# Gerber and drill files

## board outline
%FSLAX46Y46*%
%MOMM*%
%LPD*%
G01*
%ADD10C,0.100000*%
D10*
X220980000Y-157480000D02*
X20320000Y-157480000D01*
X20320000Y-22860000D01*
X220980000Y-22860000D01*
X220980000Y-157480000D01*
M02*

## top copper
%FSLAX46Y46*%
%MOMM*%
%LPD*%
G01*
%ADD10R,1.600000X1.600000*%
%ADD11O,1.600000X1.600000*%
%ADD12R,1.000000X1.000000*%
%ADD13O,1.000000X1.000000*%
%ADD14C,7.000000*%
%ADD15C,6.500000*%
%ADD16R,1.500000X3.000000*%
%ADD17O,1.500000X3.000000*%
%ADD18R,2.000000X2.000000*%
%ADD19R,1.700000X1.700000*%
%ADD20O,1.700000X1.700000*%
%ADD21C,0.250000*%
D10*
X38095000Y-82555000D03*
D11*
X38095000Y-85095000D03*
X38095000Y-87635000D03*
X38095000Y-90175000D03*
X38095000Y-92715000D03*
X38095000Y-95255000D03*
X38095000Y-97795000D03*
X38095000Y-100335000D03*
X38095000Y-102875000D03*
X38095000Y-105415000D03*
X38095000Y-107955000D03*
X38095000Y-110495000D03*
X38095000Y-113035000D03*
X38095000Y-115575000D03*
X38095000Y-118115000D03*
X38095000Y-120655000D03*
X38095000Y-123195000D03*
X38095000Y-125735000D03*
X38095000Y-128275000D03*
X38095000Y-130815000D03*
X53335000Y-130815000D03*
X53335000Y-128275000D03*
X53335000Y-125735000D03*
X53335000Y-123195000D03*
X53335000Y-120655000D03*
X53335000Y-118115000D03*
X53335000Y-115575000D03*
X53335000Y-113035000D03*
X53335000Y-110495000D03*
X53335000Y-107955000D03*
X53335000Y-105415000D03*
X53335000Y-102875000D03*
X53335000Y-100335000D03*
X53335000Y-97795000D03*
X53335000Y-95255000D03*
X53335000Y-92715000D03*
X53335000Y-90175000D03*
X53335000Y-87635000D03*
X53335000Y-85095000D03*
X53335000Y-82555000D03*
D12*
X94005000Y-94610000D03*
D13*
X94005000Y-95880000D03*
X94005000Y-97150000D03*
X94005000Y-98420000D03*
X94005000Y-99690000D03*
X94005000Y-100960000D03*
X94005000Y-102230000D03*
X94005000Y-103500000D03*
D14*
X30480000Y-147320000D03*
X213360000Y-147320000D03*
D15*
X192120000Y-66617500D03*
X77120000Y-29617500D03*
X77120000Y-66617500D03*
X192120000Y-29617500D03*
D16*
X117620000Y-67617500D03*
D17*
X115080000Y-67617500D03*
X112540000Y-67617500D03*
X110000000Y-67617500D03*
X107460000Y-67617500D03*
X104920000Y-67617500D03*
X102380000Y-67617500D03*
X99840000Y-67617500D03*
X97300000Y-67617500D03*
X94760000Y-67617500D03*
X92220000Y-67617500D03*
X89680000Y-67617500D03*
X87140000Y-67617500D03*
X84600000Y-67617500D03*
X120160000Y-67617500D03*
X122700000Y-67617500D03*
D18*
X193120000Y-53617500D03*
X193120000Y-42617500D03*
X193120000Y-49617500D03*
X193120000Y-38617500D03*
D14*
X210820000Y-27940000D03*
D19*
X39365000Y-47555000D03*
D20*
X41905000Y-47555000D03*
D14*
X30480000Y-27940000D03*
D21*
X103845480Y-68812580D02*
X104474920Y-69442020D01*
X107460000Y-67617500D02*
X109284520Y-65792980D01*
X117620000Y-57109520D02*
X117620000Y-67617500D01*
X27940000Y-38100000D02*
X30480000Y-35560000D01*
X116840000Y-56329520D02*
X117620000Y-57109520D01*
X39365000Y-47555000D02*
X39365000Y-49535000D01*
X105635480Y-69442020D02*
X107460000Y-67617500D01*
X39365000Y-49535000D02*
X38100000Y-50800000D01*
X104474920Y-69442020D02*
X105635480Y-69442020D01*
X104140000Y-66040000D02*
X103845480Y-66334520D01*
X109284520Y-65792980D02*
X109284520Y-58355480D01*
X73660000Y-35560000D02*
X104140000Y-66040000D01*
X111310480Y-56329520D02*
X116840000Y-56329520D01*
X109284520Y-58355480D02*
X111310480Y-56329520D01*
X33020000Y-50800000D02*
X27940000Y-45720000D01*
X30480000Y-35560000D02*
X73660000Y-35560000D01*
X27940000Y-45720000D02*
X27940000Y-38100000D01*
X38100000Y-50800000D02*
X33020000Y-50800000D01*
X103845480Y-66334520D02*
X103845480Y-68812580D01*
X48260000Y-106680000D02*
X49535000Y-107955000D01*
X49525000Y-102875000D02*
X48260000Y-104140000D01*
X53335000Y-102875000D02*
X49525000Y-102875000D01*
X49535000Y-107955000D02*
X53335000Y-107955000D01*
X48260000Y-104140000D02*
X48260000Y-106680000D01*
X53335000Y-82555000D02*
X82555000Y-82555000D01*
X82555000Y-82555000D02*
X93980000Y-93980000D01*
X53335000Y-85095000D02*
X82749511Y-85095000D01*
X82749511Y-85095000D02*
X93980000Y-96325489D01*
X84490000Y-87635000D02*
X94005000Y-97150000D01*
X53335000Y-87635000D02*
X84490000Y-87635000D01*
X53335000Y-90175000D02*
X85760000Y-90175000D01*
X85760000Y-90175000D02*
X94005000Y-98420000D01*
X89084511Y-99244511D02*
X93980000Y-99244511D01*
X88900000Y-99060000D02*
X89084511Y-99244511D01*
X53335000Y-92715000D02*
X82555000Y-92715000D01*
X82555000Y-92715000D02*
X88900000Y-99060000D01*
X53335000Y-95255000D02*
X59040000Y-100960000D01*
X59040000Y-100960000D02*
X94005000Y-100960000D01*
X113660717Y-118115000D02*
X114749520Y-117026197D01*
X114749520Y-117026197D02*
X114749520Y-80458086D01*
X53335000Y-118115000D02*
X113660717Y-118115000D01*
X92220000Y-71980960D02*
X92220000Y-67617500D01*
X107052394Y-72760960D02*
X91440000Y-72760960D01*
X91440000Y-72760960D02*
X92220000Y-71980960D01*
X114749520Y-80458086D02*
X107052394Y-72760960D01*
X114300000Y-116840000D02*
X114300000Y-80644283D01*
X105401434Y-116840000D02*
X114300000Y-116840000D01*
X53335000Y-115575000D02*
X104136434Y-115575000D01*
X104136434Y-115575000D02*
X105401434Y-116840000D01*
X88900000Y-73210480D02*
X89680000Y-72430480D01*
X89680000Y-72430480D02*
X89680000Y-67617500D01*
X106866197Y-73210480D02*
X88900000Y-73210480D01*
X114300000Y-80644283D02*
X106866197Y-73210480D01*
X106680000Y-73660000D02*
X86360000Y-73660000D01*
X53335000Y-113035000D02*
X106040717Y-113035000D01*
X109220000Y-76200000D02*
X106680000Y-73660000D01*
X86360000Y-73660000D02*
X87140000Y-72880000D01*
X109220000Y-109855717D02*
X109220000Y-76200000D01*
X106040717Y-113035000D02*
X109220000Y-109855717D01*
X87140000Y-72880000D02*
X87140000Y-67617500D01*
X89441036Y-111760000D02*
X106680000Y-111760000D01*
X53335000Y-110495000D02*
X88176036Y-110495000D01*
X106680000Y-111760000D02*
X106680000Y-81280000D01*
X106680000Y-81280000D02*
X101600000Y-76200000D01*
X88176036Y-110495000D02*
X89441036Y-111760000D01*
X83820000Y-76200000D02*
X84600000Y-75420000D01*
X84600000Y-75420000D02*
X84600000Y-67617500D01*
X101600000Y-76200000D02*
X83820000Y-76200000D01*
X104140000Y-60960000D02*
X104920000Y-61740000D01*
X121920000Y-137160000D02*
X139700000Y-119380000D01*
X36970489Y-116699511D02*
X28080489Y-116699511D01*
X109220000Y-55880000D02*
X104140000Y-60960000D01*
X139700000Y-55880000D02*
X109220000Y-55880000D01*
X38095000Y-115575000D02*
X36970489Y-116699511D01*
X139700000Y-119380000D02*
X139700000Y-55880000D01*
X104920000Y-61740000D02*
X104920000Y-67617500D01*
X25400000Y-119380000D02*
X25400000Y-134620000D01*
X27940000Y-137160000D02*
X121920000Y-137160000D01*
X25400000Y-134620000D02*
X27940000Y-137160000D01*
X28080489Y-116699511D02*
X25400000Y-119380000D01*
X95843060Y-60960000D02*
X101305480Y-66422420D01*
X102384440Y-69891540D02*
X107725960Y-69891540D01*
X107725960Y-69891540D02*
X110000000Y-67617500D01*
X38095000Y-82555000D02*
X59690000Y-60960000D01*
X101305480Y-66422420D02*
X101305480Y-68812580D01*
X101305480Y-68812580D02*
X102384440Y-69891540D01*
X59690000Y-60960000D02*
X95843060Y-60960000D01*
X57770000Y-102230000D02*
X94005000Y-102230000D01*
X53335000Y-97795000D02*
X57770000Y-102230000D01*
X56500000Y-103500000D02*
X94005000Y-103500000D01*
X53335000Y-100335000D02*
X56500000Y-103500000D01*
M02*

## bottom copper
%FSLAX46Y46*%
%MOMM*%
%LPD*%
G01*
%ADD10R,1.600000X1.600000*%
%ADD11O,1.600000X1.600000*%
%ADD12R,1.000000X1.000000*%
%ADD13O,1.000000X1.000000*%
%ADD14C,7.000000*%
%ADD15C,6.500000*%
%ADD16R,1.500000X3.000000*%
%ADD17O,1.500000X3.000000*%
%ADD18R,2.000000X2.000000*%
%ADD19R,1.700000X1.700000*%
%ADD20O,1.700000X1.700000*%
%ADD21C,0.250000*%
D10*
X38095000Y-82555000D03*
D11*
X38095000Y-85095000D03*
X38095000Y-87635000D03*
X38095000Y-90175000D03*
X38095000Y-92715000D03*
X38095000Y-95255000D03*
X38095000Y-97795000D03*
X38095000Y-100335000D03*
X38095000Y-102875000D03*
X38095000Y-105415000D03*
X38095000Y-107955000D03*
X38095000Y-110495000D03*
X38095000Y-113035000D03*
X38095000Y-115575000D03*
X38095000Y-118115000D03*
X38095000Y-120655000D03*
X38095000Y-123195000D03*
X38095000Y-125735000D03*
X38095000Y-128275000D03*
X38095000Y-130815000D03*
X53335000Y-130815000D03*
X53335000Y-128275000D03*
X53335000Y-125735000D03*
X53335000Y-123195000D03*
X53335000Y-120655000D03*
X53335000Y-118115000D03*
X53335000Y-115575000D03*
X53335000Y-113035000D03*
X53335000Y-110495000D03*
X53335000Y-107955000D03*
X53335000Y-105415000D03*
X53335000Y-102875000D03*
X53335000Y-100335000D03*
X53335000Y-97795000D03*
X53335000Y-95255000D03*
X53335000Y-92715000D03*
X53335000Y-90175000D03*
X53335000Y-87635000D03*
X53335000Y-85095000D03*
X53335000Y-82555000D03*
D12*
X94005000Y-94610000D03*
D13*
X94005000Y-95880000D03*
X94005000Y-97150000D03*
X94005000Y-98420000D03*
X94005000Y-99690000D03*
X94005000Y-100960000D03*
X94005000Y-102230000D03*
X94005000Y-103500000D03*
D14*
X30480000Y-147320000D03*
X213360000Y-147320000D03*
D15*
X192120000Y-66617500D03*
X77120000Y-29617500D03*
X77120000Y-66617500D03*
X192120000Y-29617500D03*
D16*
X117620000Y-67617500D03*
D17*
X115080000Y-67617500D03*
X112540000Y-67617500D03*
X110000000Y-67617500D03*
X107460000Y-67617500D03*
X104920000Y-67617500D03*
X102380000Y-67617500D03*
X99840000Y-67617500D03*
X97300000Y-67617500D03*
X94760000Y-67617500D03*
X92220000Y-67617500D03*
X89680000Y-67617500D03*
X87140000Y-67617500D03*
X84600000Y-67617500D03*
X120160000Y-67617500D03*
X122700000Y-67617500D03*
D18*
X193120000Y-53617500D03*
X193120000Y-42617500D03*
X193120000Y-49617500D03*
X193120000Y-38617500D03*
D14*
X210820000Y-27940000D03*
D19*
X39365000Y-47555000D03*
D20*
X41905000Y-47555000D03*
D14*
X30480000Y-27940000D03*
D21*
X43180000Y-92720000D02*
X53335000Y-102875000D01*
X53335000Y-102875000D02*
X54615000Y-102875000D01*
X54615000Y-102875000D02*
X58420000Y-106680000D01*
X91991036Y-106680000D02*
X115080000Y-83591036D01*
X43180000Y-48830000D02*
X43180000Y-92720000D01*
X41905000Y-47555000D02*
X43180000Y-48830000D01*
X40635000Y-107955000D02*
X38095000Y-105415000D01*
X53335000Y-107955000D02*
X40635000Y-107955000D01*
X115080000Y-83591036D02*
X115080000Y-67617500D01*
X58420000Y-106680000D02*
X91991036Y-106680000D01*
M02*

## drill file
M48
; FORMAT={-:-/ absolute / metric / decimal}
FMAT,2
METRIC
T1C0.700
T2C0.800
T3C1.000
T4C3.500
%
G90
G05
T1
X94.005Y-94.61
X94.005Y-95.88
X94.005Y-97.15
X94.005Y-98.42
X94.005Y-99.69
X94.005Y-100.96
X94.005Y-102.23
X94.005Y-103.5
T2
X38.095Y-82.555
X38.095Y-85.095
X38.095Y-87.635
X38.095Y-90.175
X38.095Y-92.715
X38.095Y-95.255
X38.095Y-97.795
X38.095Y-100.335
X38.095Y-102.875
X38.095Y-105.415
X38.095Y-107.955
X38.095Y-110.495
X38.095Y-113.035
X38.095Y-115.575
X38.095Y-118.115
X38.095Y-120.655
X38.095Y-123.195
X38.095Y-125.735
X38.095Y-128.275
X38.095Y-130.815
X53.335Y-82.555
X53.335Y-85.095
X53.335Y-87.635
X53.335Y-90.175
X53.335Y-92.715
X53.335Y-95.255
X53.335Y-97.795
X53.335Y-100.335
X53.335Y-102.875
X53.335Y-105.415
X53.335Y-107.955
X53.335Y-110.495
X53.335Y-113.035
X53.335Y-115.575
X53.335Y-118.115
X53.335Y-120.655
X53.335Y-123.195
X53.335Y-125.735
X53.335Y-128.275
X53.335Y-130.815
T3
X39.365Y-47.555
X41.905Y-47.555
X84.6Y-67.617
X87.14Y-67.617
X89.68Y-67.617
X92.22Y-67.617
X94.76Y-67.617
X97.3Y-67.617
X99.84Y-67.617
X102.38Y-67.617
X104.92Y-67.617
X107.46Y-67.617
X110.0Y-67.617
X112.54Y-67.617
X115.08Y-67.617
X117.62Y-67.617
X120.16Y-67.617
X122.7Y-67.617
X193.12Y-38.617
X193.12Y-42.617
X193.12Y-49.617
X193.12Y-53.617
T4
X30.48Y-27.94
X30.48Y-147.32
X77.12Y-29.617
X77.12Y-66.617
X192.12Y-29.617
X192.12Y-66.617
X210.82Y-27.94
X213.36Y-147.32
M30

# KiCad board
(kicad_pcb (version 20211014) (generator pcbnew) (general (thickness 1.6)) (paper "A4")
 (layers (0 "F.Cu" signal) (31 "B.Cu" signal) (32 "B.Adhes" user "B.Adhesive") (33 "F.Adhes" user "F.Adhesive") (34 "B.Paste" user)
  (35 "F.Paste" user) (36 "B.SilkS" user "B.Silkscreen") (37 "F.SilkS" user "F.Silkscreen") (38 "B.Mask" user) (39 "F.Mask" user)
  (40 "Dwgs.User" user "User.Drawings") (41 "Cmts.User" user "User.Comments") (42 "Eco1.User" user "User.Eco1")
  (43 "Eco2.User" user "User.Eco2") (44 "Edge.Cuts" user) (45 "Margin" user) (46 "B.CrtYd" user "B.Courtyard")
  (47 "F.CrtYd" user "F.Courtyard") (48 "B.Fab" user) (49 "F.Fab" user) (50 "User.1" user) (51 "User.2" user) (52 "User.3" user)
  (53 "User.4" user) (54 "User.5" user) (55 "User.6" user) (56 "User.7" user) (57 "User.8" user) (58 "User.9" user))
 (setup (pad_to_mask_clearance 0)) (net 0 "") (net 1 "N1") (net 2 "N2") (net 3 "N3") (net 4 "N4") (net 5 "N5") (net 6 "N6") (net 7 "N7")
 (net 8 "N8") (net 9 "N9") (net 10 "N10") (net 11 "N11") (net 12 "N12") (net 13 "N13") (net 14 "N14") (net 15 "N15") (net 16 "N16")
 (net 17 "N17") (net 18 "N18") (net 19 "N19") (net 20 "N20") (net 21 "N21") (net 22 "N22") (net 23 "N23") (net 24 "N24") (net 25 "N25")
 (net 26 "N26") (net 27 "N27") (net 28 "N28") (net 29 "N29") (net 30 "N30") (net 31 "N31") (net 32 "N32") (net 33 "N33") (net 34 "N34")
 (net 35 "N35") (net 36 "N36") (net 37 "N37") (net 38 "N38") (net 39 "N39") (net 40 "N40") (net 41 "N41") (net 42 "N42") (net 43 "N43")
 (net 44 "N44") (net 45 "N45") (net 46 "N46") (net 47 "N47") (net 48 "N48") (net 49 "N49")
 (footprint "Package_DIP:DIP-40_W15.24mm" (layer "F.Cu") (at 38.095 82.555)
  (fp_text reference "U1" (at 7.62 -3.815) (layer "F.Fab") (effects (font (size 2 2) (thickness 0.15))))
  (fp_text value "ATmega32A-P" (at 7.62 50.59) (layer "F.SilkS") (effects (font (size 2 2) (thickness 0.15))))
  (pad "1" thru_hole rect (at 0 0) (size 1.6 1.6) (drill 0.8) (layers *.Cu *.Mask) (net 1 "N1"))
  (pad "2" thru_hole oval (at 0 2.54) (size 1.6 1.6) (drill 0.8) (layers *.Cu *.Mask) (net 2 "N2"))
  (pad "3" thru_hole oval (at 0 5.08) (size 1.6 1.6) (drill 0.8) (layers *.Cu *.Mask) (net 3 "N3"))
  (pad "4" thru_hole oval (at 0 7.62) (size 1.6 1.6) (drill 0.8) (layers *.Cu *.Mask) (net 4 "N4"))
  (pad "5" thru_hole oval (at 0 10.16) (size 1.6 1.6) (drill 0.8) (layers *.Cu *.Mask) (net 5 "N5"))
  (pad "6" thru_hole oval (at 0 12.7) (size 1.6 1.6) (drill 0.8) (layers *.Cu *.Mask) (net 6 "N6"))
  (pad "7" thru_hole oval (at 0 15.24) (size 1.6 1.6) (drill 0.8) (layers *.Cu *.Mask) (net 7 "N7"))
  (pad "8" thru_hole oval (at 0 17.78) (size 1.6 1.6) (drill 0.8) (layers *.Cu *.Mask) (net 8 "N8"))
  (pad "9" thru_hole oval (at 0 20.32) (size 1.6 1.6) (drill 0.8) (layers *.Cu *.Mask) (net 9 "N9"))
  (pad "10" thru_hole oval (at 0 22.86) (size 1.6 1.6) (drill 0.8) (layers *.Cu *.Mask) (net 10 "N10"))
  (pad "11" thru_hole oval (at 0 25.4) (size 1.6 1.6) (drill 0.8) (layers *.Cu *.Mask) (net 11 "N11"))
  (pad "12" thru_hole oval (at 0 27.94) (size 1.6 1.6) (drill 0.8) (layers *.Cu *.Mask) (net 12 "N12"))
  (pad "13" thru_hole oval (at 0 30.48) (size 1.6 1.6) (drill 0.8) (layers *.Cu *.Mask) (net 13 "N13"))
  (pad "14" thru_hole oval (at 0 33.02) (size 1.6 1.6) (drill 0.8) (layers *.Cu *.Mask) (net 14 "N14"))
  (pad "15" thru_hole oval (at 0 35.56) (size 1.6 1.6) (drill 0.8) (layers *.Cu *.Mask) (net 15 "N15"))
  (pad "16" thru_hole oval (at 0 38.1) (size 1.6 1.6) (drill 0.8) (layers *.Cu *.Mask) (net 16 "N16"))
  (pad "17" thru_hole oval (at 0 40.64) (size 1.6 1.6) (drill 0.8) (layers *.Cu *.Mask) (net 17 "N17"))
  (pad "18" thru_hole oval (at 0 43.18) (size 1.6 1.6) (drill 0.8) (layers *.Cu *.Mask) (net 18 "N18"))
  (pad "19" thru_hole oval (at 0 45.72) (size 1.6 1.6) (drill 0.8) (layers *.Cu *.Mask) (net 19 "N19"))
  (pad "20" thru_hole oval (at 0 48.26) (size 1.6 1.6) (drill 0.8) (layers *.Cu *.Mask) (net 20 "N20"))
  (pad "21" thru_hole oval (at 15.24 48.26) (size 1.6 1.6) (drill 0.8) (layers *.Cu *.Mask) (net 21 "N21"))
  (pad "22" thru_hole oval (at 15.24 45.72) (size 1.6 1.6) (drill 0.8) (layers *.Cu *.Mask) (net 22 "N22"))
  (pad "23" thru_hole oval (at 15.24 43.18) (size 1.6 1.6) (drill 0.8) (layers *.Cu *.Mask) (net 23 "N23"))
  (pad "24" thru_hole oval (at 15.24 40.64) (size 1.6 1.6) (drill 0.8) (layers *.Cu *.Mask) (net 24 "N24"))
  (pad "25" thru_hole oval (at 15.24 38.1) (size 1.6 1.6) (drill 0.8) (layers *.Cu *.Mask) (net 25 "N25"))
  (pad "26" thru_hole oval (at 15.24 35.56) (size 1.6 1.6) (drill 0.8) (layers *.Cu *.Mask) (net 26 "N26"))
  (pad "27" thru_hole oval (at 15.24 33.02) (size 1.6 1.6) (drill 0.8) (layers *.Cu *.Mask) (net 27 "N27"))
  (pad "28" thru_hole oval (at 15.24 30.48) (size 1.6 1.6) (drill 0.8) (layers *.Cu *.Mask) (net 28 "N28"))
  (pad "29" thru_hole oval (at 15.24 27.94) (size 1.6 1.6) (drill 0.8) (layers *.Cu *.Mask) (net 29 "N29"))
  (pad "30" thru_hole oval (at 15.24 25.4) (size 1.6 1.6) (drill 0.8) (layers *.Cu *.Mask) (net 10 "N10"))
  (pad "31" thru_hole oval (at 15.24 22.86) (size 1.6 1.6) (drill 0.8) (layers *.Cu *.Mask) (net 11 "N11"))
  (pad "32" thru_hole oval (at 15.24 20.32) (size 1.6 1.6) (drill 0.8) (layers *.Cu *.Mask) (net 10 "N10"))
  (pad "33" thru_hole oval (at 15.24 17.78) (size 1.6 1.6) (drill 0.8) (layers *.Cu *.Mask) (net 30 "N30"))
  (pad "34" thru_hole oval (at 15.24 15.24) (size 1.6 1.6) (drill 0.8) (layers *.Cu *.Mask) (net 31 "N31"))
  (pad "35" thru_hole oval (at 15.24 12.7) (size 1.6 1.6) (drill 0.8) (layers *.Cu *.Mask) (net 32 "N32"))
  (pad "36" thru_hole oval (at 15.24 10.16) (size 1.6 1.6) (drill 0.8) (layers *.Cu *.Mask) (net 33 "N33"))
  (pad "37" thru_hole oval (at 15.24 7.62) (size 1.6 1.6) (drill 0.8) (layers *.Cu *.Mask) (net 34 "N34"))
  (pad "38" thru_hole oval (at 15.24 5.08) (size 1.6 1.6) (drill 0.8) (layers *.Cu *.Mask) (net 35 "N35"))
  (pad "39" thru_hole oval (at 15.24 2.54) (size 1.6 1.6) (drill 0.8) (layers *.Cu *.Mask) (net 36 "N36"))
  (pad "40" thru_hole oval (at 15.24 0) (size 1.6 1.6) (drill 0.8) (layers *.Cu *.Mask) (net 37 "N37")))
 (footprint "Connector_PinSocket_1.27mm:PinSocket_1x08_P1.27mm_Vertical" (layer "F.Cu") (at 94.005 94.61)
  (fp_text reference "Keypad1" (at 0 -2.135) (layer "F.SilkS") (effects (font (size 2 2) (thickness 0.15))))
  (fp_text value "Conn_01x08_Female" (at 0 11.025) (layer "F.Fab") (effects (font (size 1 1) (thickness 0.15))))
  (pad "1" thru_hole rect (at 0 0) (size 1 1) (drill 0.7) (layers *.Cu *.Mask) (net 37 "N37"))
  (pad "2" thru_hole oval (at 0 1.27) (size 1 1) (drill 0.7) (layers *.Cu *.Mask) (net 36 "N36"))
  (pad "3" thru_hole oval (at 0 2.54) (size 1 1) (drill 0.7) (layers *.Cu *.Mask) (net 35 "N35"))
  (pad "4" thru_hole oval (at 0 3.81) (size 1 1) (drill 0.7) (layers *.Cu *.Mask) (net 34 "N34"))
  (pad "5" thru_hole oval (at 0 5.08) (size 1 1) (drill 0.7) (layers *.Cu *.Mask) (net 33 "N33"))
  (pad "6" thru_hole oval (at 0 6.35) (size 1 1) (drill 0.7) (layers *.Cu *.Mask) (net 32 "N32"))
  (pad "7" thru_hole oval (at 0 7.62) (size 1 1) (drill 0.7) (layers *.Cu *.Mask) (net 31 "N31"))
  (pad "8" thru_hole oval (at 0 8.89) (size 1 1) (drill 0.7) (layers *.Cu *.Mask) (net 30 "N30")))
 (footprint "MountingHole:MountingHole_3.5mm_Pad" (layer "F.Cu") (at 30.48 147.32)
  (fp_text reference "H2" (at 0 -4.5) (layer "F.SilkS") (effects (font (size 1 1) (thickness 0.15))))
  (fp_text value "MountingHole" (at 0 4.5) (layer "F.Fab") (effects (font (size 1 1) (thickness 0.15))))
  (pad "1" thru_hole circle (at 0 0) (size 7 7) (drill 3.5) (layers *.Cu *.Mask)))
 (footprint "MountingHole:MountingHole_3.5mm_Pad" (layer "F.Cu") (at 213.36 147.32)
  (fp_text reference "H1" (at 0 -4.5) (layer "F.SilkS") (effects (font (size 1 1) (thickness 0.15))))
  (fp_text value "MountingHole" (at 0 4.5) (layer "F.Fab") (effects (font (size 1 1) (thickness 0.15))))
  (pad "1" thru_hole circle (at 0 0) (size 7 7) (drill 3.5) (layers *.Cu *.Mask)))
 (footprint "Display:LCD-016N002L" (layer "F.Cu") (at 117.62 67.6175 180)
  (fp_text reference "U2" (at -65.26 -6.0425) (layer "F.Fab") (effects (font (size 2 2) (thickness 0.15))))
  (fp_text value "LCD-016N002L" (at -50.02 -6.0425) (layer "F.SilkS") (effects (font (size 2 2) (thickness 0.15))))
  (pad "" thru_hole circle (at -74.5 1) (size 6.5 6.5) (drill 3.5) (layers *.Cu *.Mask))
  (pad "" thru_hole circle (at 40.5 38) (size 6.5 6.5) (drill 3.5) (layers *.Cu *.Mask))
  (pad "" thru_hole circle (at 40.5 1) (size 6.5 6.5) (drill 3.5) (layers *.Cu *.Mask))
  (pad "" thru_hole circle (at -74.5 38) (size 6.5 6.5) (drill 3.5) (layers *.Cu *.Mask))
  (pad "1" thru_hole rect (at 0 0) (size 1.5 3) (drill 1) (layers *.Cu *.Mask) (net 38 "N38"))
  (pad "2" thru_hole oval (at 2.54 0) (size 1.5 3) (drill 1) (layers *.Cu *.Mask) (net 10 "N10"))
  (pad "3" thru_hole oval (at 5.08 0) (size 1.5 3) (drill 1) (layers *.Cu *.Mask) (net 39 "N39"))
  (pad "4" thru_hole oval (at 7.62 0) (size 1.5 3) (drill 1) (layers *.Cu *.Mask) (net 1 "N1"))
  (pad "5" thru_hole oval (at 10.16 0) (size 1.5 3) (drill 1) (layers *.Cu *.Mask) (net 38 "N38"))
  (pad "6" thru_hole oval (at 12.7 0) (size 1.5 3) (drill 1) (layers *.Cu *.Mask) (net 14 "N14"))
  (pad "7" thru_hole oval (at 15.24 0) (size 1.5 3) (drill 1) (layers *.Cu *.Mask) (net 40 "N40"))
  (pad "8" thru_hole oval (at 17.78 0) (size 1.5 3) (drill 1) (layers *.Cu *.Mask) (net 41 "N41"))
  (pad "9" thru_hole oval (at 20.32 0) (size 1.5 3) (drill 1) (layers *.Cu *.Mask) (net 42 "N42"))
  (pad "10" thru_hole oval (at 22.86 0) (size 1.5 3) (drill 1) (layers *.Cu *.Mask) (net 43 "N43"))
  (pad "11" thru_hole oval (at 25.4 0) (size 1.5 3) (drill 1) (layers *.Cu *.Mask) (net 26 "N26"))
  (pad "12" thru_hole oval (at 27.94 0) (size 1.5 3) (drill 1) (layers *.Cu *.Mask) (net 27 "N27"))
  (pad "13" thru_hole oval (at 30.48 0) (size 1.5 3) (drill 1) (layers *.Cu *.Mask) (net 28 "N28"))
  (pad "14" thru_hole oval (at 33.02 0) (size 1.5 3) (drill 1) (layers *.Cu *.Mask) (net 29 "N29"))
  (pad "15" thru_hole oval (at -2.54 0) (size 1.5 3) (drill 1) (layers *.Cu *.Mask) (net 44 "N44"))
  (pad "16" thru_hole oval (at -5.08 0) (size 1.5 3) (drill 1) (layers *.Cu *.Mask) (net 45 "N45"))
  (pad "A1" thru_hole rect (at -75.5 14) (size 2 2) (drill 1) (layers *.Cu *.Mask) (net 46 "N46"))
  (pad "A2" thru_hole rect (at -75.5 25) (size 2 2) (drill 1) (layers *.Cu *.Mask) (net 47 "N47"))
  (pad "K1" thru_hole rect (at -75.5 18) (size 2 2) (drill 1) (layers *.Cu *.Mask) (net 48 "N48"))
  (pad "K2" thru_hole rect (at -75.5 29) (size 2 2) (drill 1) (layers *.Cu *.Mask) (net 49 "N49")))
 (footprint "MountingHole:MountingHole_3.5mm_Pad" (layer "F.Cu") (at 210.82 27.94)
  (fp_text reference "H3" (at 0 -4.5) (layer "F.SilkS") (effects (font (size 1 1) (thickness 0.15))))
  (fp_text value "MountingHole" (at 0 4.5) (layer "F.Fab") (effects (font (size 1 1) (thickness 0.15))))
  (pad "1" thru_hole circle (at 0 0) (size 7 7) (drill 3.5) (layers *.Cu *.Mask)))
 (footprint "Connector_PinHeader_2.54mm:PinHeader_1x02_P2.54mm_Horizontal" (layer "F.Cu") (at 39.365 47.555 90)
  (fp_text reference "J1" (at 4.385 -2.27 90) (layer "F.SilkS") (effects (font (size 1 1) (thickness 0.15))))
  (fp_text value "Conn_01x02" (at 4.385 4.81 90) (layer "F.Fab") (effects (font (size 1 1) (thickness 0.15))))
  (pad "1" thru_hole rect (at 0 0 90) (size 1.7 1.7) (drill 1) (layers *.Cu *.Mask) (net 38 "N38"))
  (pad "2" thru_hole oval (at 0 2.54 90) (size 1.7 1.7) (drill 1) (layers *.Cu *.Mask) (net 10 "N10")))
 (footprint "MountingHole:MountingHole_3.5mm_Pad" (layer "F.Cu") (at 30.48 27.94)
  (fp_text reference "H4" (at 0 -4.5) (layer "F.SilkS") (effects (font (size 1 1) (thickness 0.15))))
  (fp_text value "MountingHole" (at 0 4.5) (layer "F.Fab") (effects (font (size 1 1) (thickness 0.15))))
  (pad "1" thru_hole circle (at 0 0) (size 7 7) (drill 3.5) (layers *.Cu *.Mask)))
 (gr_poly (pts (xy 220.98 157.48) (xy 20.32 157.48) (xy 20.32 22.86) (xy 220.98 22.86)) (layer "Edge.Cuts") (width 0.1) (fill none))
 (segment (start 103.84548 68.81258) (end 104.47492 69.44202) (width 0.25) (layer "F.Cu") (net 38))
 (segment (start 107.46 67.6175) (end 109.28452 65.79298) (width 0.25) (layer "F.Cu") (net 38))
 (segment (start 117.62 57.10952) (end 117.62 67.6175) (width 0.25) (layer "F.Cu") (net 38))
 (segment (start 27.94 38.1) (end 30.48 35.56) (width 0.25) (layer "F.Cu") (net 38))
 (segment (start 116.84 56.32952) (end 117.62 57.10952) (width 0.25) (layer "F.Cu") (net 38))
 (segment (start 39.365 47.555) (end 39.365 49.535) (width 0.25) (layer "F.Cu") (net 38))
 (segment (start 105.63548 69.44202) (end 107.46 67.6175) (width 0.25) (layer "F.Cu") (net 38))
 (segment (start 39.365 49.535) (end 38.1 50.8) (width 0.25) (layer "F.Cu") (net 38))
 (segment (start 104.47492 69.44202) (end 105.63548 69.44202) (width 0.25) (layer "F.Cu") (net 38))
 (segment (start 104.14 66.04) (end 103.84548 66.33452) (width 0.25) (layer "F.Cu") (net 38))
 (segment (start 109.28452 65.79298) (end 109.28452 58.35548) (width 0.25) (layer "F.Cu") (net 38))
 (segment (start 73.66 35.56) (end 104.14 66.04) (width 0.25) (layer "F.Cu") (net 38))
 (segment (start 111.31048 56.32952) (end 116.84 56.32952) (width 0.25) (layer "F.Cu") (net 38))
 (segment (start 109.28452 58.35548) (end 111.31048 56.32952) (width 0.25) (layer "F.Cu") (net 38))
 (segment (start 33.02 50.8) (end 27.94 45.72) (width 0.25) (layer "F.Cu") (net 38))
 (segment (start 30.48 35.56) (end 73.66 35.56) (width 0.25) (layer "F.Cu") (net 38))
 (segment (start 27.94 45.72) (end 27.94 38.1) (width 0.25) (layer "F.Cu") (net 38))
 (segment (start 38.1 50.8) (end 33.02 50.8) (width 0.25) (layer "F.Cu") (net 38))
 (segment (start 103.84548 66.33452) (end 103.84548 68.81258) (width 0.25) (layer "F.Cu") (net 38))
 (segment (start 48.26 106.68) (end 49.535 107.955) (width 0.25) (layer "F.Cu") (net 10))
 (segment (start 49.525 102.875) (end 48.26 104.14) (width 0.25) (layer "F.Cu") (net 10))
 (segment (start 53.335 102.875) (end 49.525 102.875) (width 0.25) (layer "F.Cu") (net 10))
 (segment (start 49.535 107.955) (end 53.335 107.955) (width 0.25) (layer "F.Cu") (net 10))
 (segment (start 48.26 104.14) (end 48.26 106.68) (width 0.25) (layer "F.Cu") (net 10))
 (segment (start 43.18 92.72) (end 53.335 102.875) (width 0.25) (layer "B.Cu") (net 10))
 (segment (start 53.335 102.875) (end 54.615 102.875) (width 0.25) (layer "B.Cu") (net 10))
 (segment (start 54.615 102.875) (end 58.42 106.68) (width 0.25) (layer "B.Cu") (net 10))
 (segment (start 91.991036 106.68) (end 115.08 83.591036) (width 0.25) (layer "B.Cu") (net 10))
 (segment (start 43.18 48.83) (end 43.18 92.72) (width 0.25) (layer "B.Cu") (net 10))
 (segment (start 41.905 47.555) (end 43.18 48.83) (width 0.25) (layer "B.Cu") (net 10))
 (segment (start 40.635 107.955) (end 38.095 105.415) (width 0.25) (layer "B.Cu") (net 10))
 (segment (start 53.335 107.955) (end 40.635 107.955) (width 0.25) (layer "B.Cu") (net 10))
 (segment (start 115.08 83.591036) (end 115.08 67.6175) (width 0.25) (layer "B.Cu") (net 10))
 (segment (start 58.42 106.68) (end 91.991036 106.68) (width 0.25) (layer "B.Cu") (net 10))
 (segment (start 53.335 82.555) (end 82.555 82.555) (width 0.25) (layer "F.Cu") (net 37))
 (segment (start 82.555 82.555) (end 93.98 93.98) (width 0.25) (layer "F.Cu") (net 37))
 (segment (start 53.335 85.095) (end 82.749511 85.095) (width 0.25) (layer "F.Cu") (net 36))
 (segment (start 82.749511 85.095) (end 93.98 96.325489) (width 0.25) (layer "F.Cu") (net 36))
 (segment (start 84.49 87.635) (end 94.005 97.15) (width 0.25) (layer "F.Cu") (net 35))
 (segment (start 53.335 87.635) (end 84.49 87.635) (width 0.25) (layer "F.Cu") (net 35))
 (segment (start 53.335 90.175) (end 85.76 90.175) (width 0.25) (layer "F.Cu") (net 34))
 (segment (start 85.76 90.175) (end 94.005 98.42) (width 0.25) (layer "F.Cu") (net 34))
 (segment (start 89.084511 99.244511) (end 93.98 99.244511) (width 0.25) (layer "F.Cu") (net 33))
 (segment (start 88.9 99.06) (end 89.084511 99.244511) (width 0.25) (layer "F.Cu") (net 33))
 (segment (start 53.335 92.715) (end 82.555 92.715) (width 0.25) (layer "F.Cu") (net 33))
 (segment (start 82.555 92.715) (end 88.9 99.06) (width 0.25) (layer "F.Cu") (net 33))
 (segment (start 53.335 95.255) (end 59.04 100.96) (width 0.25) (layer "F.Cu") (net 32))
 (segment (start 59.04 100.96) (end 94.005 100.96) (width 0.25) (layer "F.Cu") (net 32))
 (segment (start 113.660717 118.115) (end 114.74952 117.026197) (width 0.25) (layer "F.Cu") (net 26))
 (segment (start 114.74952 117.026197) (end 114.74952 80.458086) (width 0.25) (layer "F.Cu") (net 26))
 (segment (start 53.335 118.115) (end 113.660717 118.115) (width 0.25) (layer "F.Cu") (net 26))
 (segment (start 92.22 71.98096) (end 92.22 67.6175) (width 0.25) (layer "F.Cu") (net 26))
 (segment (start 107.052394 72.76096) (end 91.44 72.76096) (width 0.25) (layer "F.Cu") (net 26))
 (segment (start 91.44 72.76096) (end 92.22 71.98096) (width 0.25) (layer "F.Cu") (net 26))
 (segment (start 114.74952 80.458086) (end 107.052394 72.76096) (width 0.25) (layer "F.Cu") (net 26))
 (segment (start 114.3 116.84) (end 114.3 80.644283) (width 0.25) (layer "F.Cu") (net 27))
 (segment (start 105.401434 116.84) (end 114.3 116.84) (width 0.25) (layer "F.Cu") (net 27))
 (segment (start 53.335 115.575) (end 104.136434 115.575) (width 0.25) (layer "F.Cu") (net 27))
 (segment (start 104.136434 115.575) (end 105.401434 116.84) (width 0.25) (layer "F.Cu") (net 27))
 (segment (start 88.9 73.21048) (end 89.68 72.43048) (width 0.25) (layer "F.Cu") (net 27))
 (segment (start 89.68 72.43048) (end 89.68 67.6175) (width 0.25) (layer "F.Cu") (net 27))
 (segment (start 106.866197 73.21048) (end 88.9 73.21048) (width 0.25) (layer "F.Cu") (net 27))
 (segment (start 114.3 80.644283) (end 106.866197 73.21048) (width 0.25) (layer "F.Cu") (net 27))
 (segment (start 106.68 73.66) (end 86.36 73.66) (width 0.25) (layer "F.Cu") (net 28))
 (segment (start 53.335 113.035) (end 106.040717 113.035) (width 0.25) (layer "F.Cu") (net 28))
 (segment (start 109.22 76.2) (end 106.68 73.66) (width 0.25) (layer "F.Cu") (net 28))
 (segment (start 86.36 73.66) (end 87.14 72.88) (width 0.25) (layer "F.Cu") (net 28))
 (segment (start 109.22 109.855717) (end 109.22 76.2) (width 0.25) (layer "F.Cu") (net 28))
 (segment (start 106.040717 113.035) (end 109.22 109.855717) (width 0.25) (layer "F.Cu") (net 28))
 (segment (start 87.14 72.88) (end 87.14 67.6175) (width 0.25) (layer "F.Cu") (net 28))
 (segment (start 89.441036 111.76) (end 106.68 111.76) (width 0.25) (layer "F.Cu") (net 29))
 (segment (start 53.335 110.495) (end 88.176036 110.495) (width 0.25) (layer "F.Cu") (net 29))
 (segment (start 106.68 111.76) (end 106.68 81.28) (width 0.25) (layer "F.Cu") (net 29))
 (segment (start 106.68 81.28) (end 101.6 76.2) (width 0.25) (layer "F.Cu") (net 29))
 (segment (start 88.176036 110.495) (end 89.441036 111.76) (width 0.25) (layer "F.Cu") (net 29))
 (segment (start 83.82 76.2) (end 84.6 75.42) (width 0.25) (layer "F.Cu") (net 29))
 (segment (start 84.6 75.42) (end 84.6 67.6175) (width 0.25) (layer "F.Cu") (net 29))
 (segment (start 101.6 76.2) (end 83.82 76.2) (width 0.25) (layer "F.Cu") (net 29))
 (segment (start 104.14 60.96) (end 104.92 61.74) (width 0.25) (layer "F.Cu") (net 14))
 (segment (start 121.92 137.16) (end 139.7 119.38) (width 0.25) (layer "F.Cu") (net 14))
 (segment (start 36.970489 116.699511) (end 28.080489 116.699511) (width 0.25) (layer "F.Cu") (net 14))
 (segment (start 109.22 55.88) (end 104.14 60.96) (width 0.25) (layer "F.Cu") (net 14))
 (segment (start 139.7 55.88) (end 109.22 55.88) (width 0.25) (layer "F.Cu") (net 14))
 (segment (start 38.095 115.575) (end 36.970489 116.699511) (width 0.25) (layer "F.Cu") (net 14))
 (segment (start 139.7 119.38) (end 139.7 55.88) (width 0.25) (layer "F.Cu") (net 14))
 (segment (start 104.92 61.74) (end 104.92 67.6175) (width 0.25) (layer "F.Cu") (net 14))
 (segment (start 25.4 119.38) (end 25.4 134.62) (width 0.25) (layer "F.Cu") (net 14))
 (segment (start 27.94 137.16) (end 121.92 137.16) (width 0.25) (layer "F.Cu") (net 14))
 (segment (start 25.4 134.62) (end 27.94 137.16) (width 0.25) (layer "F.Cu") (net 14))
 (segment (start 28.080489 116.699511) (end 25.4 119.38) (width 0.25) (layer "F.Cu") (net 14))
 (segment (start 95.84306 60.96) (end 101.30548 66.42242) (width 0.25) (layer "F.Cu") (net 1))
 (segment (start 102.38444 69.89154) (end 107.72596 69.89154) (width 0.25) (layer "F.Cu") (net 1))
 (segment (start 107.72596 69.89154) (end 110 67.6175) (width 0.25) (layer "F.Cu") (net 1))
 (segment (start 38.095 82.555) (end 59.69 60.96) (width 0.25) (layer "F.Cu") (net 1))
 (segment (start 101.30548 66.42242) (end 101.30548 68.81258) (width 0.25) (layer "F.Cu") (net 1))
 (segment (start 101.30548 68.81258) (end 102.38444 69.89154) (width 0.25) (layer "F.Cu") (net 1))
 (segment (start 59.69 60.96) (end 95.84306 60.96) (width 0.25) (layer "F.Cu") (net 1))
 (segment (start 57.77 102.23) (end 94.005 102.23) (width 0.25) (layer "F.Cu") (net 31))
 (segment (start 53.335 97.795) (end 57.77 102.23) (width 0.25) (layer "F.Cu") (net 31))
 (segment (start 56.5 103.5) (end 94.005 103.5) (width 0.25) (layer "F.Cu") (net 30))
 (segment (start 53.335 100.335) (end 56.5 103.5) (width 0.25) (layer "F.Cu") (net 30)))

